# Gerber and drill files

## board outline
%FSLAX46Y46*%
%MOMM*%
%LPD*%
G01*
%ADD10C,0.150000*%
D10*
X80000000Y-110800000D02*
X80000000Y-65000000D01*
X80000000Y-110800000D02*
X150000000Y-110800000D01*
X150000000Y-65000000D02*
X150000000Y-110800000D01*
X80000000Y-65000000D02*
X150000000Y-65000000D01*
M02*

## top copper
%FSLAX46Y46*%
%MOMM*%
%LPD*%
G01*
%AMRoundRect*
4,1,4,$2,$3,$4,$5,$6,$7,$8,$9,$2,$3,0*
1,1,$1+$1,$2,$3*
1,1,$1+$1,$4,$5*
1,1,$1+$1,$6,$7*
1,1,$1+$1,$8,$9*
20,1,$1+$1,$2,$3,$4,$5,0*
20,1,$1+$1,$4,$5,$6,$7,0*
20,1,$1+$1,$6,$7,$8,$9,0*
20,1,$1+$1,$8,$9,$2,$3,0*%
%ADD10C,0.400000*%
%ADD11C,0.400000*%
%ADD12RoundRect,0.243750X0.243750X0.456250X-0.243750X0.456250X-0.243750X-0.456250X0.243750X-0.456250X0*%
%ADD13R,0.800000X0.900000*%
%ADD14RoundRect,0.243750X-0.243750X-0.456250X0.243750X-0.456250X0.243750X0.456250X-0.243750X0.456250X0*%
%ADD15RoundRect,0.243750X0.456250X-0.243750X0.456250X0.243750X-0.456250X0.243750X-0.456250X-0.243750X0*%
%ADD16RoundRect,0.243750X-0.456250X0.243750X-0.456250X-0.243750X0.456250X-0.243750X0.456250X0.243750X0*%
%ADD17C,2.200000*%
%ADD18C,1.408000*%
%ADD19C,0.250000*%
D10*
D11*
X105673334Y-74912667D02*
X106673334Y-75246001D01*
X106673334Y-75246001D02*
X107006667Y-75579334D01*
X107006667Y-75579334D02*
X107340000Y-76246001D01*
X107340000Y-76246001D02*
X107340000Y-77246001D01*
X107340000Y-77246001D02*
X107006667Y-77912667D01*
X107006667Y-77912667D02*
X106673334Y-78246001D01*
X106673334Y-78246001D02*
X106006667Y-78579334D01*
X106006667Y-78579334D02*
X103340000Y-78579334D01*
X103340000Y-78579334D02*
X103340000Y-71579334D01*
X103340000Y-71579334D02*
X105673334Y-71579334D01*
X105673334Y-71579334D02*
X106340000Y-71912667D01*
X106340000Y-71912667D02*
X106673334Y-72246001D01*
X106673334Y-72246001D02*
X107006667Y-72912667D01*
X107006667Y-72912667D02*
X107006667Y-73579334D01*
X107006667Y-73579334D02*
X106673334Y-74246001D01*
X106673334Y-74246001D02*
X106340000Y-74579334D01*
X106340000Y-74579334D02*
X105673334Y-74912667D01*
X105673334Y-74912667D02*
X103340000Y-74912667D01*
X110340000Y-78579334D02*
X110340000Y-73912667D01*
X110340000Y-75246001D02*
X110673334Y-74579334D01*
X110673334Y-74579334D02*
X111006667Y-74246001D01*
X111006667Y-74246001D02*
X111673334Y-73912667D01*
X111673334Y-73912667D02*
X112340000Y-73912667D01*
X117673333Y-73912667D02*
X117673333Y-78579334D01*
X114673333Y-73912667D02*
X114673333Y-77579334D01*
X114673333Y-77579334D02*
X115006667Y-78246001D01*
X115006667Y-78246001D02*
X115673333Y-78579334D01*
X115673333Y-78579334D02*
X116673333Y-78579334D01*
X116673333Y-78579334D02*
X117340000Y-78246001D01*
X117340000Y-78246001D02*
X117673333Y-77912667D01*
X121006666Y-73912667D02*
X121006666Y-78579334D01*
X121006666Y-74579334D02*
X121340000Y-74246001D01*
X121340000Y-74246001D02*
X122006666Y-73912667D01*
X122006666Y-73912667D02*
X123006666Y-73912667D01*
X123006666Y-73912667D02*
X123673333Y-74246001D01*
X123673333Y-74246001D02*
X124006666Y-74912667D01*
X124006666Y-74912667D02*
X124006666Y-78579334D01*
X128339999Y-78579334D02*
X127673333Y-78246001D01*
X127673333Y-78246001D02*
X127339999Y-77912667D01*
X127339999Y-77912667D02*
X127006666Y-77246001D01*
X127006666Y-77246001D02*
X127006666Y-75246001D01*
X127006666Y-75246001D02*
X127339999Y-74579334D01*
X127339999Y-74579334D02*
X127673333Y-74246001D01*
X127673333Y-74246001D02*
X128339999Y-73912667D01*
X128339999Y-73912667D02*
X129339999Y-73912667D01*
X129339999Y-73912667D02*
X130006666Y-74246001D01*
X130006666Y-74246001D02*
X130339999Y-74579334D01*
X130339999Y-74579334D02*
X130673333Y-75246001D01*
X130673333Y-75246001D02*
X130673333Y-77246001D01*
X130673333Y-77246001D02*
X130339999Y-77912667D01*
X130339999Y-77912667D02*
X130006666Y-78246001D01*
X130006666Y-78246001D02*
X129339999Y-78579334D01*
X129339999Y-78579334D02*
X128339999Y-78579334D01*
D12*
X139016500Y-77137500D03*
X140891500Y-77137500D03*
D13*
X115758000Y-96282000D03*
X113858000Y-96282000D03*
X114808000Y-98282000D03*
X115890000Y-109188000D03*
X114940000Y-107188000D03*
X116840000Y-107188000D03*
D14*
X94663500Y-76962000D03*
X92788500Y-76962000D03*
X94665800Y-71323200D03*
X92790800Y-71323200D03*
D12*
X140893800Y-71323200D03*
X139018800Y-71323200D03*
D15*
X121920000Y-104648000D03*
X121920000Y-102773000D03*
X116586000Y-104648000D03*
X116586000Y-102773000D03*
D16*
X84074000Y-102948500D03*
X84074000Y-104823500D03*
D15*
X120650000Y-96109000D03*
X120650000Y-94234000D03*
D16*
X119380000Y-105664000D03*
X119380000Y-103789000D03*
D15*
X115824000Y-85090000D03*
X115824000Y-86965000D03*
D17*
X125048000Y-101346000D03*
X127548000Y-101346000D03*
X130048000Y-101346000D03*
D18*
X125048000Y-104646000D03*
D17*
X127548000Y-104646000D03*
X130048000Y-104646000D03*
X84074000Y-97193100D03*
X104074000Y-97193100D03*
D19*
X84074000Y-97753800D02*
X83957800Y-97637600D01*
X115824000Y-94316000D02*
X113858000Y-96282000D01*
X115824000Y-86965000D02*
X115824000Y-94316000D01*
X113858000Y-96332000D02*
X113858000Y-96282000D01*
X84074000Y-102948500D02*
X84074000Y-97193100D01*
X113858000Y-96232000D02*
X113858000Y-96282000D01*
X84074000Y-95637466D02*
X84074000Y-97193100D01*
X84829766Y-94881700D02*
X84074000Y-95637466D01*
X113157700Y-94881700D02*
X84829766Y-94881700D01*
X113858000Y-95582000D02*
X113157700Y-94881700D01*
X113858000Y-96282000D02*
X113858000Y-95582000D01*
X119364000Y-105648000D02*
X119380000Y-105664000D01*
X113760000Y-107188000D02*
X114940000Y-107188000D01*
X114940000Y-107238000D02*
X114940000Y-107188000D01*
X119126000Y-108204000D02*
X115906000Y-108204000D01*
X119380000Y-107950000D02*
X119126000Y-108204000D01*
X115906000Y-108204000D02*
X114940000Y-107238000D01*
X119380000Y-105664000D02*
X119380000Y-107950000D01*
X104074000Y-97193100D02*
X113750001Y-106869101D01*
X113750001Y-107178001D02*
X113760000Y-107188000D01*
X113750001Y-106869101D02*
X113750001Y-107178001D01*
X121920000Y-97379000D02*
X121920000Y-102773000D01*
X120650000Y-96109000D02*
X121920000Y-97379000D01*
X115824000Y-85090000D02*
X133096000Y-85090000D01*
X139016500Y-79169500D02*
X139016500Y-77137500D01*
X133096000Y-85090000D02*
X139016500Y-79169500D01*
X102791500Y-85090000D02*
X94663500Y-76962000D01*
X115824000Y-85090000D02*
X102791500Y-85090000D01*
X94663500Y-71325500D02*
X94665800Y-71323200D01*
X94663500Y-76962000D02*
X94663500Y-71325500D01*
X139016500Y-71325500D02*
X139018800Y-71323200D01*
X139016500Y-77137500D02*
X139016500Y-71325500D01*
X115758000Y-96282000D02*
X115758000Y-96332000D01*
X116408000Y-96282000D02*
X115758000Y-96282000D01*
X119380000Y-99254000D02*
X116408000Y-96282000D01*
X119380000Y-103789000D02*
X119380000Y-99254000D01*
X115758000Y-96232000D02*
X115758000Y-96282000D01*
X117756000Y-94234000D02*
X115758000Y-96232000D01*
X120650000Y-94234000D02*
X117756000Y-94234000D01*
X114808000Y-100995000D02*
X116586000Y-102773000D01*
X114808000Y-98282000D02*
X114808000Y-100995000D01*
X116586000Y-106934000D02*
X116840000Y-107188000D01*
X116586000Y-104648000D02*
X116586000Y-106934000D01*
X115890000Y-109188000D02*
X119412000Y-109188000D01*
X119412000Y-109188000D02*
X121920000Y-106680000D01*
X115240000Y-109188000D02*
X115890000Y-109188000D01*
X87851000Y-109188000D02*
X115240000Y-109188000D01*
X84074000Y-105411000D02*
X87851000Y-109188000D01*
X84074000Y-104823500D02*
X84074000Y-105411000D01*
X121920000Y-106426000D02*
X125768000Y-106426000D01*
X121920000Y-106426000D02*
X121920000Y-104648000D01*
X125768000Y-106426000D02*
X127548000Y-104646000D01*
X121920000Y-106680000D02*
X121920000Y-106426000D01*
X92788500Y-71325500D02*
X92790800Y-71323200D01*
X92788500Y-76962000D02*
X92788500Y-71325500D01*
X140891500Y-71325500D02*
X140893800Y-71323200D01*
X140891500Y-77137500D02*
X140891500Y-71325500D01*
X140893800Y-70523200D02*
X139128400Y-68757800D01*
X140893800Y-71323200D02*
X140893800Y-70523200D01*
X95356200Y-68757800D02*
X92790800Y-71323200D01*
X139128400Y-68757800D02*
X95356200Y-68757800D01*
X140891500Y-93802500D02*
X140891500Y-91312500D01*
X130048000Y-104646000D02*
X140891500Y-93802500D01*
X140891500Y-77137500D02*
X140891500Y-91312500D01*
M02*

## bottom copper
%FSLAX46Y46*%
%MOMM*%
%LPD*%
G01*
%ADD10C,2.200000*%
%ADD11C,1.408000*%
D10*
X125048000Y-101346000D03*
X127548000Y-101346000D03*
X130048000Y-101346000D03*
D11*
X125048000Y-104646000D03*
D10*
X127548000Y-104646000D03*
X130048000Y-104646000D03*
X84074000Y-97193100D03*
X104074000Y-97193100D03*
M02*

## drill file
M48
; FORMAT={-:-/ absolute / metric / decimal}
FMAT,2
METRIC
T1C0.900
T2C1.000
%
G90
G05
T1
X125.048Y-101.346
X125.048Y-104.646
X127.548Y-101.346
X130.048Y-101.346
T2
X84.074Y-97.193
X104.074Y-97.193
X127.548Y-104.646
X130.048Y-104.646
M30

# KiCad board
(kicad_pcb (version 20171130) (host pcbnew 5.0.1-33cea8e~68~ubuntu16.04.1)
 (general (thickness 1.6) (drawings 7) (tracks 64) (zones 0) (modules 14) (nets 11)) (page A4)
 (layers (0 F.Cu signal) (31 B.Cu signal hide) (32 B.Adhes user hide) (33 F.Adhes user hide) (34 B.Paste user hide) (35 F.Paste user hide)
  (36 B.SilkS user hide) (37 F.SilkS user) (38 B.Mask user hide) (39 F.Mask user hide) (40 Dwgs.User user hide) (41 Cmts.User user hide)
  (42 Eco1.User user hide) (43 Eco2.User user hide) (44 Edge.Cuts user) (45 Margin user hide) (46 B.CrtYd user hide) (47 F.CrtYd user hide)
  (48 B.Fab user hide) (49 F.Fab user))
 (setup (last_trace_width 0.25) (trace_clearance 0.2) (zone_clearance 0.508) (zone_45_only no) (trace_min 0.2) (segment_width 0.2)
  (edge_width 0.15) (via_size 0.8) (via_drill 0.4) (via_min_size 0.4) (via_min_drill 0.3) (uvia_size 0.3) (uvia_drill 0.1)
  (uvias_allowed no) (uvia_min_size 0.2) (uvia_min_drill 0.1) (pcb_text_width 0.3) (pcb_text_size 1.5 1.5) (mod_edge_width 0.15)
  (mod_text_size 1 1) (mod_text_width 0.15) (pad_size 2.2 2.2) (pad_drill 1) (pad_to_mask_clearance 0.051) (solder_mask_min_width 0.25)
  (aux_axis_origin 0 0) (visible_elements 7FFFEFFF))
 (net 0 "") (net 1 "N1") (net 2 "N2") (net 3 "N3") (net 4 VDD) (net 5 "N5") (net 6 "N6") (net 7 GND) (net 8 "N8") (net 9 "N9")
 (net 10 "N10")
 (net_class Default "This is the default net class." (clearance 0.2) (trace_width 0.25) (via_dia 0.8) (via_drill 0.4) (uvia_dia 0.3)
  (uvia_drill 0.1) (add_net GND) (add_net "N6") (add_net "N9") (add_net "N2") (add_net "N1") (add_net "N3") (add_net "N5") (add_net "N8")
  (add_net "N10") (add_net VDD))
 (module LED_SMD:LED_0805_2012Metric (layer F.Cu) (at 139.954 77.1375 180)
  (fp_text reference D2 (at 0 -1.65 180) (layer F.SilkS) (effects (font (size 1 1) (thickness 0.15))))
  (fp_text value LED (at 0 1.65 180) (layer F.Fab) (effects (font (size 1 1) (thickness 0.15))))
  (pad 2 smd roundrect (at 0.9375 0 180) (size 0.975 1.4) (layers F.Cu F.Paste F.Mask) (roundrect_rratio 0.25) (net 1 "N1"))
  (pad 1 smd roundrect (at -0.9375 0 180) (size 0.975 1.4) (layers F.Cu F.Paste F.Mask) (roundrect_rratio 0.25) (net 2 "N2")))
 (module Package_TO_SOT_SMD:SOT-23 (layer F.Cu) (at 114.808 97.282 270)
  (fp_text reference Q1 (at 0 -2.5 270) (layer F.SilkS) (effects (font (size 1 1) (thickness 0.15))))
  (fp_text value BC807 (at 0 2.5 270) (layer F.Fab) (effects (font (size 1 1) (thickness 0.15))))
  (pad 1 smd rect (at -1 -0.95 270) (size 0.9 0.8) (layers F.Cu F.Paste F.Mask) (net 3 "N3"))
  (pad 2 smd rect (at -1 0.95 270) (size 0.9 0.8) (layers F.Cu F.Paste F.Mask) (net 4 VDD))
  (pad 3 smd rect (at 1 0 270) (size 0.9 0.8) (layers F.Cu F.Paste F.Mask) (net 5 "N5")))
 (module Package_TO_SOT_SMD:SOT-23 (layer F.Cu) (at 115.89 108.188 270)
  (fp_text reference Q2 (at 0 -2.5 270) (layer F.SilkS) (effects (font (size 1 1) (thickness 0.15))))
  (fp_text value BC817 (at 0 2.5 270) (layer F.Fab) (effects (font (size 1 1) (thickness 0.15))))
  (pad 3 smd rect (at 1 0 270) (size 0.9 0.8) (layers F.Cu F.Paste F.Mask) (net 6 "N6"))
  (pad 2 smd rect (at -1 0.95 270) (size 0.9 0.8) (layers F.Cu F.Paste F.Mask) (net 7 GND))
  (pad 1 smd rect (at -1 -0.95 270) (size 0.9 0.8) (layers F.Cu F.Paste F.Mask) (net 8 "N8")))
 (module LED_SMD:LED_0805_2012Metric (layer F.Cu) (at 93.726 76.962)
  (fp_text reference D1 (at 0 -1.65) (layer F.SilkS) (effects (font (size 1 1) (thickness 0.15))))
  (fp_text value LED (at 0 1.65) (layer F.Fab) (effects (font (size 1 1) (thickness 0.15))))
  (pad 2 smd roundrect (at 0.9375 0) (size 0.975 1.4) (layers F.Cu F.Paste F.Mask) (roundrect_rratio 0.25) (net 1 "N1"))
  (pad 1 smd roundrect (at -0.9375 0) (size 0.975 1.4) (layers F.Cu F.Paste F.Mask) (roundrect_rratio 0.25) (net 2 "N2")))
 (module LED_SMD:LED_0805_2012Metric (layer F.Cu) (at 93.7283 71.3232)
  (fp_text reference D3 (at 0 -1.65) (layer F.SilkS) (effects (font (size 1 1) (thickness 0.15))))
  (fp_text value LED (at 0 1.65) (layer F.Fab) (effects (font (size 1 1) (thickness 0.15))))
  (pad 2 smd roundrect (at 0.9375 0) (size 0.975 1.4) (layers F.Cu F.Paste F.Mask) (roundrect_rratio 0.25) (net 1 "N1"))
  (pad 1 smd roundrect (at -0.9375 0) (size 0.975 1.4) (layers F.Cu F.Paste F.Mask) (roundrect_rratio 0.25) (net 2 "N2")))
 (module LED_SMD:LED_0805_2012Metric (layer F.Cu) (at 139.9563 71.3232 180)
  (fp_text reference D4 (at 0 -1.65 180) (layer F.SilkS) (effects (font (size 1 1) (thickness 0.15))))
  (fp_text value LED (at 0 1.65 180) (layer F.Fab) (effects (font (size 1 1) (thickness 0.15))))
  (pad 1 smd roundrect (at -0.9375 0 180) (size 0.975 1.4) (layers F.Cu F.Paste F.Mask) (roundrect_rratio 0.25) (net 2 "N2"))
  (pad 2 smd roundrect (at 0.9375 0 180) (size 0.975 1.4) (layers F.Cu F.Paste F.Mask) (roundrect_rratio 0.25) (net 1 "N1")))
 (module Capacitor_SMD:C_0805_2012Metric (layer F.Cu) (at 121.92 103.7105 90)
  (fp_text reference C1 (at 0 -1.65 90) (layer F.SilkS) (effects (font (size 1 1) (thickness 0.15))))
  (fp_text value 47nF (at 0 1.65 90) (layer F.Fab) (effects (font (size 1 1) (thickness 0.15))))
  (pad 1 smd roundrect (at -0.9375 0 90) (size 0.975 1.4) (layers F.Cu F.Paste F.Mask) (roundrect_rratio 0.25) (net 6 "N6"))
  (pad 2 smd roundrect (at 0.9375 0 90) (size 0.975 1.4) (layers F.Cu F.Paste F.Mask) (roundrect_rratio 0.25) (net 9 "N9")))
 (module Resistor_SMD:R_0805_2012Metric (layer F.Cu) (at 116.586 103.7105 90)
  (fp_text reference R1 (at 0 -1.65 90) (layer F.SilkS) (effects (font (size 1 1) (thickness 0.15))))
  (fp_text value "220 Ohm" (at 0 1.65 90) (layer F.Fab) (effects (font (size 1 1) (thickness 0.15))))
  (pad 1 smd roundrect (at -0.9375 0 90) (size 0.975 1.4) (layers F.Cu F.Paste F.Mask) (roundrect_rratio 0.25) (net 8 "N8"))
  (pad 2 smd roundrect (at 0.9375 0 90) (size 0.975 1.4) (layers F.Cu F.Paste F.Mask) (roundrect_rratio 0.25) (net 5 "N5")))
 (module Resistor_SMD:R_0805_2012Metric (layer F.Cu) (at 84.074 103.886 270)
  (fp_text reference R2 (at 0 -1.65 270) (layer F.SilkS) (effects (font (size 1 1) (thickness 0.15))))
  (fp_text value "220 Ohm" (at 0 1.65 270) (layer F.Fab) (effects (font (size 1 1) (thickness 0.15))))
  (pad 1 smd roundrect (at -0.9375 0 270) (size 0.975 1.4) (layers F.Cu F.Paste F.Mask) (roundrect_rratio 0.25) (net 4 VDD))
  (pad 2 smd roundrect (at 0.9375 0 270) (size 0.975 1.4) (layers F.Cu F.Paste F.Mask) (roundrect_rratio 0.25) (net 6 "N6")))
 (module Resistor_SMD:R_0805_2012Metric (layer F.Cu) (at 120.65 95.1715 90)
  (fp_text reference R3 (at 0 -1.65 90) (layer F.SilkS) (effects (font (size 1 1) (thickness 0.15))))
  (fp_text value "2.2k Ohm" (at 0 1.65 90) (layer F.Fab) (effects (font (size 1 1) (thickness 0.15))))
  (pad 1 smd roundrect (at -0.9375 0 90) (size 0.975 1.4) (layers F.Cu F.Paste F.Mask) (roundrect_rratio 0.25) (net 9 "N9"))
  (pad 2 smd roundrect (at 0.9375 0 90) (size 0.975 1.4) (layers F.Cu F.Paste F.Mask) (roundrect_rratio 0.25) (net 3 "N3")))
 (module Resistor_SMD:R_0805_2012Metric (layer F.Cu) (at 119.38 104.7265 270)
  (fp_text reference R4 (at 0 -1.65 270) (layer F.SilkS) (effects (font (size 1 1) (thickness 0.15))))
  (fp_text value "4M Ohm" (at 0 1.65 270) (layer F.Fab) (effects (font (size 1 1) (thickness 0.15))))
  (pad 2 smd roundrect (at 0.9375 0 270) (size 0.975 1.4) (layers F.Cu F.Paste F.Mask) (roundrect_rratio 0.25) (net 7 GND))
  (pad 1 smd roundrect (at -0.9375 0 270) (size 0.975 1.4) (layers F.Cu F.Paste F.Mask) (roundrect_rratio 0.25) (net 3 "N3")))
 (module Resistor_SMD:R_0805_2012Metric (layer F.Cu) (at 115.824 86.0275 90)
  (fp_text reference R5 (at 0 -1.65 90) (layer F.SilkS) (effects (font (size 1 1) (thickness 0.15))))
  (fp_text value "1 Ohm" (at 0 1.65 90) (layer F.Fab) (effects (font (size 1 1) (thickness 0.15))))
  (pad 2 smd roundrect (at 0.9375 0 90) (size 0.975 1.4) (layers F.Cu F.Paste F.Mask) (roundrect_rratio 0.25) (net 1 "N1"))
  (pad 1 smd roundrect (at -0.9375 0 90) (size 0.975 1.4) (layers F.Cu F.Paste F.Mask) (roundrect_rratio 0.25) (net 4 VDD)))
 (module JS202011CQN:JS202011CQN (layer F.Cu) (at 127.548 102.996 180)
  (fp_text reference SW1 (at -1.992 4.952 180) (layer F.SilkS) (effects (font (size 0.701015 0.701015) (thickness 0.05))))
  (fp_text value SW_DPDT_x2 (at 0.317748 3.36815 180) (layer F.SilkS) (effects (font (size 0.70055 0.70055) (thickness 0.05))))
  (pad 6 thru_hole circle (at 2.5 1.65 270) (size 2.2 2.2) (drill 0.9) (layers *.Cu *.Mask))
  (pad 5 thru_hole circle (at 0 1.65 270) (size 2.2 2.2) (drill 0.9) (layers *.Cu *.Mask))
  (pad 4 thru_hole circle (at -2.5 1.65 270) (size 2.2 2.2) (drill 0.9) (layers *.Cu *.Mask))
  (pad 3 thru_hole circle (at 2.5 -1.65 270) (size 1.408 1.408) (drill 0.9) (layers *.Cu *.Mask) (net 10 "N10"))
  (pad 2 thru_hole circle (at 0 -1.65 270) (size 2.2 2.2) (drill 1) (layers *.Cu *.Mask) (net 6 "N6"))
  (pad 1 thru_hole circle (at -2.5 -1.65 270) (size 2.2 2.2) (drill 1) (layers *.Cu *.Mask) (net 2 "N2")))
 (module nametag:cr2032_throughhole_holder (layer F.Cu) (at 84.074 97.1931)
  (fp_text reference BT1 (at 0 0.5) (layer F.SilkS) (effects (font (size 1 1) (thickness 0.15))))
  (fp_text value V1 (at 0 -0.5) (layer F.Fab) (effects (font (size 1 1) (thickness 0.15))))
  (pad 1 thru_hole circle (at 0 0) (size 2.2 2.2) (drill 1) (layers *.Cu *.Mask) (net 4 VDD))
  (pad 2 thru_hole circle (at 20 0) (size 2.2 2.2) (drill 1) (layers *.Cu *.Mask) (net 7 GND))
  (pad 3 smd circle (at 14 0) (size 3.25 3.25) (layers F.Paste F.Mask)))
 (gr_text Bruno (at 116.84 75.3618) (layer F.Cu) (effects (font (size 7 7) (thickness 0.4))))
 (gr_line (start 80 110.8) (end 80 65) (layer Edge.Cuts) (width 0.15))
 (gr_line (start 80 110.8) (end 150 110.8) (layer Edge.Cuts) (width 0.15))
 (gr_line (start 150 65) (end 150 110.8) (layer Edge.Cuts) (width 0.15))
 (gr_line (start 80 65) (end 150 65) (layer Edge.Cuts) (width 0.15))
 (segment (start 84.074 97.7538) (end 83.9578 97.6376) (width 0.25) (layer F.Cu) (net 4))
 (segment (start 115.824 94.316) (end 113.858 96.282) (width 0.25) (layer F.Cu) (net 4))
 (segment (start 115.824 86.965) (end 115.824 94.316) (width 0.25) (layer F.Cu) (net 4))
 (segment (start 113.858 96.332) (end 113.858 96.282) (width 0.25) (layer F.Cu) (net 4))
 (segment (start 84.074 102.9485) (end 84.074 97.1931) (width 0.25) (layer F.Cu) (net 4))
 (segment (start 113.858 96.232) (end 113.858 96.282) (width 0.25) (layer F.Cu) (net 4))
 (segment (start 84.074 95.637466) (end 84.074 97.1931) (width 0.25) (layer F.Cu) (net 4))
 (segment (start 84.829766 94.8817) (end 84.074 95.637466) (width 0.25) (layer F.Cu) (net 4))
 (segment (start 113.1577 94.8817) (end 84.829766 94.8817) (width 0.25) (layer F.Cu) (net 4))
 (segment (start 113.858 95.582) (end 113.1577 94.8817) (width 0.25) (layer F.Cu) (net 4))
 (segment (start 113.858 96.282) (end 113.858 95.582) (width 0.25) (layer F.Cu) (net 4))
 (segment (start 119.364 105.648) (end 119.38 105.664) (width 0.25) (layer F.Cu) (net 7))
 (segment (start 113.76 107.188) (end 114.94 107.188) (width 0.25) (layer F.Cu) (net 7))
 (segment (start 114.94 107.238) (end 114.94 107.188) (width 0.25) (layer F.Cu) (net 7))
 (segment (start 119.126 108.204) (end 115.906 108.204) (width 0.25) (layer F.Cu) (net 7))
 (segment (start 119.38 107.95) (end 119.126 108.204) (width 0.25) (layer F.Cu) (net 7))
 (segment (start 115.906 108.204) (end 114.94 107.238) (width 0.25) (layer F.Cu) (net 7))
 (segment (start 119.38 105.664) (end 119.38 107.95) (width 0.25) (layer F.Cu) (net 7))
 (segment (start 104.074 97.1931) (end 113.750001 106.869101) (width 0.25) (layer F.Cu) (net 7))
 (segment (start 113.750001 107.178001) (end 113.76 107.188) (width 0.25) (layer F.Cu) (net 7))
 (segment (start 113.750001 106.869101) (end 113.750001 107.178001) (width 0.25) (layer F.Cu) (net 7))
 (segment (start 121.92 97.379) (end 121.92 102.773) (width 0.25) (layer F.Cu) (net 9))
 (segment (start 120.65 96.109) (end 121.92 97.379) (width 0.25) (layer F.Cu) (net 9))
 (segment (start 115.824 85.09) (end 133.096 85.09) (width 0.25) (layer F.Cu) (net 1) (status 10))
 (segment (start 139.0165 79.1695) (end 139.0165 77.1375) (width 0.25) (layer F.Cu) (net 1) (status 20))
 (segment (start 133.096 85.09) (end 139.0165 79.1695) (width 0.25) (layer F.Cu) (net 1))
 (segment (start 102.7915 85.09) (end 94.6635 76.962) (width 0.25) (layer F.Cu) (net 1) (status 20))
 (segment (start 115.824 85.09) (end 102.7915 85.09) (width 0.25) (layer F.Cu) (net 1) (status 10))
 (segment (start 94.6635 71.3255) (end 94.6658 71.3232) (width 0.25) (layer F.Cu) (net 1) (status 30))
 (segment (start 94.6635 76.962) (end 94.6635 71.3255) (width 0.25) (layer F.Cu) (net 1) (status 30))
 (segment (start 139.0165 71.3255) (end 139.0188 71.3232) (width 0.25) (layer F.Cu) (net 1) (status 30))
 (segment (start 139.0165 77.1375) (end 139.0165 71.3255) (width 0.25) (layer F.Cu) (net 1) (status 30))
 (segment (start 115.758 96.282) (end 115.758 96.332) (width 0.25) (layer F.Cu) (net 3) (status 30))
 (segment (start 116.408 96.282) (end 115.758 96.282) (width 0.25) (layer F.Cu) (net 3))
 (segment (start 119.38 99.254) (end 116.408 96.282) (width 0.25) (layer F.Cu) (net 3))
 (segment (start 119.38 103.789) (end 119.38 99.254) (width 0.25) (layer F.Cu) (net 3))
 (segment (start 115.758 96.232) (end 115.758 96.282) (width 0.25) (layer F.Cu) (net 3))
 (segment (start 117.756 94.234) (end 115.758 96.232) (width 0.25) (layer F.Cu) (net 3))
 (segment (start 120.65 94.234) (end 117.756 94.234) (width 0.25) (layer F.Cu) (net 3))
 (segment (start 114.808 100.995) (end 116.586 102.773) (width 0.25) (layer F.Cu) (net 5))
 (segment (start 114.808 98.282) (end 114.808 100.995) (width 0.25) (layer F.Cu) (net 5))
 (segment (start 116.586 106.934) (end 116.84 107.188) (width 0.25) (layer F.Cu) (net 8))
 (segment (start 116.586 104.648) (end 116.586 106.934) (width 0.25) (layer F.Cu) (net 8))
 (segment (start 115.89 109.188) (end 119.412 109.188) (width 0.25) (layer F.Cu) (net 6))
 (segment (start 119.412 109.188) (end 121.92 106.68) (width 0.25) (layer F.Cu) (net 6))
 (segment (start 115.24 109.188) (end 115.89 109.188) (width 0.25) (layer F.Cu) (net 6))
 (segment (start 87.851 109.188) (end 115.24 109.188) (width 0.25) (layer F.Cu) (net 6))
 (segment (start 84.074 105.411) (end 87.851 109.188) (width 0.25) (layer F.Cu) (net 6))
 (segment (start 84.074 104.8235) (end 84.074 105.411) (width 0.25) (layer F.Cu) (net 6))
 (segment (start 121.92 106.426) (end 125.768 106.426) (width 0.25) (layer F.Cu) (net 6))
 (segment (start 121.92 106.426) (end 121.92 104.648) (width 0.25) (layer F.Cu) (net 6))
 (segment (start 125.768 106.426) (end 127.548 104.646) (width 0.25) (layer F.Cu) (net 6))
 (segment (start 121.92 106.68) (end 121.92 106.426) (width 0.25) (layer F.Cu) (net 6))
 (segment (start 92.7885 71.3255) (end 92.7908 71.3232) (width 0.25) (layer F.Cu) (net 2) (status 30))
 (segment (start 92.7885 76.962) (end 92.7885 71.3255) (width 0.25) (layer F.Cu) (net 2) (status 30))
 (segment (start 140.8915 71.3255) (end 140.8938 71.3232) (width 0.25) (layer F.Cu) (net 2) (status 30))
 (segment (start 140.8915 77.1375) (end 140.8915 71.3255) (width 0.25) (layer F.Cu) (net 2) (status 30))
 (segment (start 140.8938 70.5232) (end 139.1284 68.7578) (width 0.25) (layer F.Cu) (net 2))
 (segment (start 140.8938 71.3232) (end 140.8938 70.5232) (width 0.25) (layer F.Cu) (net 2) (status 10))
 (segment (start 95.3562 68.7578) (end 92.7908 71.3232) (width 0.25) (layer F.Cu) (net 2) (status 20))
 (segment (start 139.1284 68.7578) (end 95.3562 68.7578) (width 0.25) (layer F.Cu) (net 2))
 (segment (start 140.8915 93.8025) (end 140.8915 91.3125) (width 0.25) (layer F.Cu) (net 2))
 (segment (start 130.048 104.646) (end 140.8915 93.8025) (width 0.25) (layer F.Cu) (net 2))
 (segment (start 140.8915 77.1375) (end 140.8915 91.3125) (width 0.25) (layer F.Cu) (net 2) (status 10)))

